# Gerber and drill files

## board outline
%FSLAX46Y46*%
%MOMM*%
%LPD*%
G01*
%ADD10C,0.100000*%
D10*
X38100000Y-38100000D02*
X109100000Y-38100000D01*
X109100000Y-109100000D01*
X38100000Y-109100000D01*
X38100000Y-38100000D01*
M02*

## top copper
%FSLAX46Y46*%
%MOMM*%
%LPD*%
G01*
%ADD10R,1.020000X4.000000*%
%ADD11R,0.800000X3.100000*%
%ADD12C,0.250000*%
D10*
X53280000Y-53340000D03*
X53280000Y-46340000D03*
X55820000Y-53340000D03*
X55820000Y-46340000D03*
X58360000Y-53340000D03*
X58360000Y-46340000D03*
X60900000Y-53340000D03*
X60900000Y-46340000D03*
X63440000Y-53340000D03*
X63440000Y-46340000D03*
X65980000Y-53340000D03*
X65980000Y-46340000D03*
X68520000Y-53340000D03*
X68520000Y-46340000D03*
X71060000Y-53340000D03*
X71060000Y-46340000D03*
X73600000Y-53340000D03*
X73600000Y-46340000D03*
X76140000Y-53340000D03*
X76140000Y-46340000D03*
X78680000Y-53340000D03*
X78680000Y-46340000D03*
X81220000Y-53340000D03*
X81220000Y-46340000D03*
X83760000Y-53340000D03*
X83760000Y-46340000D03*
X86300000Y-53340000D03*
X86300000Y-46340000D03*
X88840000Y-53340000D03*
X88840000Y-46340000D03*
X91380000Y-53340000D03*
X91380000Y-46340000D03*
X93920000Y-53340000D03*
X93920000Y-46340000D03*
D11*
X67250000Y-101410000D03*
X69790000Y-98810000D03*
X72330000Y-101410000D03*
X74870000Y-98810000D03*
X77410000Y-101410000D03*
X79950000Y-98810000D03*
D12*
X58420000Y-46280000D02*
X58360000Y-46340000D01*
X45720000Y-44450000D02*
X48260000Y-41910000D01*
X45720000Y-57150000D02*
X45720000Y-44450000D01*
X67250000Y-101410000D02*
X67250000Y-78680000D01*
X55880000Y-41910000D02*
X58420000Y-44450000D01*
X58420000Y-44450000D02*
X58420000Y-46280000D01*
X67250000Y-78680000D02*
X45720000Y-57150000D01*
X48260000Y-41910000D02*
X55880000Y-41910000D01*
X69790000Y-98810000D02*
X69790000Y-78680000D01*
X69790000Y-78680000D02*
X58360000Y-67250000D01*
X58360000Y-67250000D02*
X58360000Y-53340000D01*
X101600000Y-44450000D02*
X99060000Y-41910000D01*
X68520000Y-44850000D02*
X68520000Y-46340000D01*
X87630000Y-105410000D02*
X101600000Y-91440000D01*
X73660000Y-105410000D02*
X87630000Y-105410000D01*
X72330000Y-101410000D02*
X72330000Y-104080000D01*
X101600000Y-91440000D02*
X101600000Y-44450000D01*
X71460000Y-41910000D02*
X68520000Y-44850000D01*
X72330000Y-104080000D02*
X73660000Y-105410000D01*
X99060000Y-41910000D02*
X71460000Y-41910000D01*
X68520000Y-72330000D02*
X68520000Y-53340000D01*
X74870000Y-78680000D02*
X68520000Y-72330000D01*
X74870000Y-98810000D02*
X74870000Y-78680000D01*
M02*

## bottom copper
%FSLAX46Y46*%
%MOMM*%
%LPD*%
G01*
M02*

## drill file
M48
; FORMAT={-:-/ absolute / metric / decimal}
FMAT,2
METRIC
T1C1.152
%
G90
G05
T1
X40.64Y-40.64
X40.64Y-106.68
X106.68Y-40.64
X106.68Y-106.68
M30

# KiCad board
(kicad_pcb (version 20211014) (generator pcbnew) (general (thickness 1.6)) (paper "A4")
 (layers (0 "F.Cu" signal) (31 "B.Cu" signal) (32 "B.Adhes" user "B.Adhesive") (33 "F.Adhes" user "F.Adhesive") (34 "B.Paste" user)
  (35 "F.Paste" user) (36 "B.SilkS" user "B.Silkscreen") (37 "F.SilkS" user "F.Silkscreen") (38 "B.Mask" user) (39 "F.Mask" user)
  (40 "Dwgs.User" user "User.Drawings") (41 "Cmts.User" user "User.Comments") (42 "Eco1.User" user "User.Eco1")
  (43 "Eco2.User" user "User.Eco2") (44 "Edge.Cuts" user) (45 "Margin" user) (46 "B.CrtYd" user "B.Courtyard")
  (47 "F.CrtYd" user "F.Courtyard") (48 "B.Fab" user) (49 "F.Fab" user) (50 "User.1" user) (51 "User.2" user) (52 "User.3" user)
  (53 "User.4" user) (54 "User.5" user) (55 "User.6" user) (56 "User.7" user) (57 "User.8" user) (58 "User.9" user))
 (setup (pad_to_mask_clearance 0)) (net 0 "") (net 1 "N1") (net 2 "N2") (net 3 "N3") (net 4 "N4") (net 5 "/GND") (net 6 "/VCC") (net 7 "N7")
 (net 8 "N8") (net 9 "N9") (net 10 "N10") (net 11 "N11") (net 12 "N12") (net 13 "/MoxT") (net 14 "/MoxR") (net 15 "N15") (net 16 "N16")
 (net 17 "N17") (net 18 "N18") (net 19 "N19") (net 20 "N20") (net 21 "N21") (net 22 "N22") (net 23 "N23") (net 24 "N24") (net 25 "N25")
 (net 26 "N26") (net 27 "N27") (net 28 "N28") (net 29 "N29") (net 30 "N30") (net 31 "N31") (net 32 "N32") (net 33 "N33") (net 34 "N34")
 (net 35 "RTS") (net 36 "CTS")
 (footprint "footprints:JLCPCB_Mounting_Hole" (layer "F.Cu") (at 106.68 40.64)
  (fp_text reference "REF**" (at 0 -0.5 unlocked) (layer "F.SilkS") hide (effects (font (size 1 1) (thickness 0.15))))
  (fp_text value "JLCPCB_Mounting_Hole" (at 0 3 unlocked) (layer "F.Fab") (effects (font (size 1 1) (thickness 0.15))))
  (pad "" np_thru_hole circle (at 0 0) (size 1.152 1.152) (drill 1.152) (layers F&B.Cu *.Mask) (solder_mask_margin 0.148)))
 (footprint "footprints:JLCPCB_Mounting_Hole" (layer "F.Cu") (at 106.68 106.68)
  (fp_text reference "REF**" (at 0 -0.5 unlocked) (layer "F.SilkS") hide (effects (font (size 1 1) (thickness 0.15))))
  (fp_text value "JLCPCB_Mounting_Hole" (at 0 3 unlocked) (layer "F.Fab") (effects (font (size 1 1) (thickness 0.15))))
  (pad "" np_thru_hole circle (at 0 0) (size 1.152 1.152) (drill 1.152) (layers F&B.Cu *.Mask) (solder_mask_margin 0.148)))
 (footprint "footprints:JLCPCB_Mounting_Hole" (layer "F.Cu") (at 40.64 40.64)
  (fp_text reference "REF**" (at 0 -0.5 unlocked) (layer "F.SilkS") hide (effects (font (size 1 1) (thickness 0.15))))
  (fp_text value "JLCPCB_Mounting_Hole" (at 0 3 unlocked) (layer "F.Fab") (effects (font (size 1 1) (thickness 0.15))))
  (pad "" np_thru_hole circle (at 0 0) (size 1.152 1.152) (drill 1.152) (layers F&B.Cu *.Mask) (solder_mask_margin 0.148)))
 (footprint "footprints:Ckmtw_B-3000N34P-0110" (layer "F.Cu") (at 53.28 53.34)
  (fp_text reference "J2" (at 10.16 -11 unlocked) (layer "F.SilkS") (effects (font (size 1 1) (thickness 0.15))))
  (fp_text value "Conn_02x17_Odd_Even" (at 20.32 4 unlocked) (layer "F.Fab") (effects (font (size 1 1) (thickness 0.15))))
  (pad "1" smd rect (at 0 0) (size 1.02 4) (layers "F.Cu" "F.Paste" "F.Mask") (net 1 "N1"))
  (pad "2" smd rect (at 0 -7) (size 1.02 4) (layers "F.Cu" "F.Paste" "F.Mask") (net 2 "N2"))
  (pad "3" smd rect (at 2.54 0) (size 1.02 4) (layers "F.Cu" "F.Paste" "F.Mask") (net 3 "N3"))
  (pad "4" smd rect (at 2.54 -7) (size 1.02 4) (layers "F.Cu" "F.Paste" "F.Mask") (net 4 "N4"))
  (pad "5" smd rect (at 5.08 0) (size 1.02 4) (layers "F.Cu" "F.Paste" "F.Mask") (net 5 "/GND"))
  (pad "6" smd rect (at 5.08 -7) (size 1.02 4) (layers "F.Cu" "F.Paste" "F.Mask") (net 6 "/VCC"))
  (pad "7" smd rect (at 7.62 0) (size 1.02 4) (layers "F.Cu" "F.Paste" "F.Mask") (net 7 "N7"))
  (pad "8" smd rect (at 7.62 -7) (size 1.02 4) (layers "F.Cu" "F.Paste" "F.Mask") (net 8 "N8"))
  (pad "9" smd rect (at 10.16 0) (size 1.02 4) (layers "F.Cu" "F.Paste" "F.Mask") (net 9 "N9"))
  (pad "10" smd rect (at 10.16 -7) (size 1.02 4) (layers "F.Cu" "F.Paste" "F.Mask") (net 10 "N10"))
  (pad "11" smd rect (at 12.7 0) (size 1.02 4) (layers "F.Cu" "F.Paste" "F.Mask") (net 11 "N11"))
  (pad "12" smd rect (at 12.7 -7) (size 1.02 4) (layers "F.Cu" "F.Paste" "F.Mask") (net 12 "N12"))
  (pad "13" smd rect (at 15.24 0) (size 1.02 4) (layers "F.Cu" "F.Paste" "F.Mask") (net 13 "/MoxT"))
  (pad "14" smd rect (at 15.24 -7) (size 1.02 4) (layers "F.Cu" "F.Paste" "F.Mask") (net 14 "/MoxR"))
  (pad "15" smd rect (at 17.78 0) (size 1.02 4) (layers "F.Cu" "F.Paste" "F.Mask") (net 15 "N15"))
  (pad "16" smd rect (at 17.78 -7) (size 1.02 4) (layers "F.Cu" "F.Paste" "F.Mask") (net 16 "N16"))
  (pad "17" smd rect (at 20.32 0) (size 1.02 4) (layers "F.Cu" "F.Paste" "F.Mask") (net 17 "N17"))
  (pad "18" smd rect (at 20.32 -7) (size 1.02 4) (layers "F.Cu" "F.Paste" "F.Mask") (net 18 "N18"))
  (pad "19" smd rect (at 22.86 0) (size 1.02 4) (layers "F.Cu" "F.Paste" "F.Mask") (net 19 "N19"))
  (pad "20" smd rect (at 22.86 -7) (size 1.02 4) (layers "F.Cu" "F.Paste" "F.Mask") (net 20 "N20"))
  (pad "21" smd rect (at 25.4 0) (size 1.02 4) (layers "F.Cu" "F.Paste" "F.Mask") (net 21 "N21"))
  (pad "22" smd rect (at 25.4 -7) (size 1.02 4) (layers "F.Cu" "F.Paste" "F.Mask") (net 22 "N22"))
  (pad "23" smd rect (at 27.94 0) (size 1.02 4) (layers "F.Cu" "F.Paste" "F.Mask") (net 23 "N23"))
  (pad "24" smd rect (at 27.94 -7) (size 1.02 4) (layers "F.Cu" "F.Paste" "F.Mask") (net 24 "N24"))
  (pad "25" smd rect (at 30.48 0) (size 1.02 4) (layers "F.Cu" "F.Paste" "F.Mask") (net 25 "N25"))
  (pad "26" smd rect (at 30.48 -7) (size 1.02 4) (layers "F.Cu" "F.Paste" "F.Mask") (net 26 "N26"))
  (pad "27" smd rect (at 33.02 0) (size 1.02 4) (layers "F.Cu" "F.Paste" "F.Mask") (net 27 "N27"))
  (pad "28" smd rect (at 33.02 -7) (size 1.02 4) (layers "F.Cu" "F.Paste" "F.Mask") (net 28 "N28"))
  (pad "29" smd rect (at 35.56 0) (size 1.02 4) (layers "F.Cu" "F.Paste" "F.Mask") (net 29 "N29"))
  (pad "30" smd rect (at 35.56 -7) (size 1.02 4) (layers "F.Cu" "F.Paste" "F.Mask") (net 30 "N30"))
  (pad "31" smd rect (at 38.1 0) (size 1.02 4) (layers "F.Cu" "F.Paste" "F.Mask") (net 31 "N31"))
  (pad "32" smd rect (at 38.1 -7) (size 1.02 4) (layers "F.Cu" "F.Paste" "F.Mask") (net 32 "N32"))
  (pad "33" smd rect (at 40.64 0) (size 1.02 4) (layers "F.Cu" "F.Paste" "F.Mask") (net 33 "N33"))
  (pad "34" smd rect (at 40.64 -7) (size 1.02 4) (layers "F.Cu" "F.Paste" "F.Mask") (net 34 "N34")))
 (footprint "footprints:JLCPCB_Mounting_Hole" (layer "F.Cu") (at 40.64 106.68)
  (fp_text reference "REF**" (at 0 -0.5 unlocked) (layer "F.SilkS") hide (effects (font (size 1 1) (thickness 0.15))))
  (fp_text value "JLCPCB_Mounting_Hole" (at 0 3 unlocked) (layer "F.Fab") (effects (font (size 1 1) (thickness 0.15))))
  (pad "" np_thru_hole circle (at 0 0) (size 1.152 1.152) (drill 1.152) (layers F&B.Cu *.Mask) (solder_mask_margin 0.148)))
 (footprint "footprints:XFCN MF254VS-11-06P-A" (layer "F.Cu") (at 67.25 101.41)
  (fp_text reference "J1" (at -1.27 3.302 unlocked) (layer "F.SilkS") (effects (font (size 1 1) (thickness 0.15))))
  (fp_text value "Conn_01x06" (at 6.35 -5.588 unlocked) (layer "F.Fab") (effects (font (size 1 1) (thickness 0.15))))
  (pad "1" smd rect (at 0 0) (size 0.8 3.1) (layers "F.Cu" "F.Paste" "F.Mask") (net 6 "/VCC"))
  (pad "2" smd rect (at 2.54 -2.6) (size 0.8 3.1) (layers "F.Cu" "F.Paste" "F.Mask") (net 5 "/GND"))
  (pad "3" smd rect (at 5.08 0) (size 0.8 3.1) (layers "F.Cu" "F.Paste" "F.Mask") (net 14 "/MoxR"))
  (pad "4" smd rect (at 7.62 -2.6) (size 0.8 3.1) (layers "F.Cu" "F.Paste" "F.Mask") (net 13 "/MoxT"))
  (pad "5" smd rect (at 10.16 0) (size 0.8 3.1) (layers "F.Cu" "F.Paste" "F.Mask") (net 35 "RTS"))
  (pad "6" smd rect (at 12.7 -2.6) (size 0.8 3.1) (layers "F.Cu" "F.Paste" "F.Mask") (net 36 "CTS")))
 (gr_rect (start 38.1 38.1) (end 109.1 109.1) (layer "Edge.Cuts") (width 0.1) (fill none))
 (segment (start 58.42 46.28) (end 58.36 46.34) (width 0.25) (layer "F.Cu") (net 6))
 (segment (start 45.72 44.45) (end 48.26 41.91) (width 0.25) (layer "F.Cu") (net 6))
 (segment (start 45.72 57.15) (end 45.72 44.45) (width 0.25) (layer "F.Cu") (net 6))
 (segment (start 67.25 101.41) (end 67.25 78.68) (width 0.25) (layer "F.Cu") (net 6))
 (segment (start 55.88 41.91) (end 58.42 44.45) (width 0.25) (layer "F.Cu") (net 6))
 (segment (start 58.42 44.45) (end 58.42 46.28) (width 0.25) (layer "F.Cu") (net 6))
 (segment (start 67.25 78.68) (end 45.72 57.15) (width 0.25) (layer "F.Cu") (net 6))
 (segment (start 48.26 41.91) (end 55.88 41.91) (width 0.25) (layer "F.Cu") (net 6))
 (segment (start 69.79 98.81) (end 69.79 78.68) (width 0.25) (layer "F.Cu") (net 5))
 (segment (start 69.79 78.68) (end 58.36 67.25) (width 0.25) (layer "F.Cu") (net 5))
 (segment (start 58.36 67.25) (end 58.36 53.34) (width 0.25) (layer "F.Cu") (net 5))
 (segment (start 101.6 44.45) (end 99.06 41.91) (width 0.25) (layer "F.Cu") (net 14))
 (segment (start 68.52 44.85) (end 68.52 46.34) (width 0.25) (layer "F.Cu") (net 14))
 (segment (start 87.63 105.41) (end 101.6 91.44) (width 0.25) (layer "F.Cu") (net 14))
 (segment (start 73.66 105.41) (end 87.63 105.41) (width 0.25) (layer "F.Cu") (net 14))
 (segment (start 72.33 101.41) (end 72.33 104.08) (width 0.25) (layer "F.Cu") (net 14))
 (segment (start 101.6 91.44) (end 101.6 44.45) (width 0.25) (layer "F.Cu") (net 14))
 (segment (start 71.46 41.91) (end 68.52 44.85) (width 0.25) (layer "F.Cu") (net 14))
 (segment (start 72.33 104.08) (end 73.66 105.41) (width 0.25) (layer "F.Cu") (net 14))
 (segment (start 99.06 41.91) (end 71.46 41.91) (width 0.25) (layer "F.Cu") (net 14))
 (segment (start 68.52 72.33) (end 68.52 53.34) (width 0.25) (layer "F.Cu") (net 13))
 (segment (start 74.87 78.68) (end 68.52 72.33) (width 0.25) (layer "F.Cu") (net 13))
 (segment (start 74.87 98.81) (end 74.87 78.68) (width 0.25) (layer "F.Cu") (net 13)))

